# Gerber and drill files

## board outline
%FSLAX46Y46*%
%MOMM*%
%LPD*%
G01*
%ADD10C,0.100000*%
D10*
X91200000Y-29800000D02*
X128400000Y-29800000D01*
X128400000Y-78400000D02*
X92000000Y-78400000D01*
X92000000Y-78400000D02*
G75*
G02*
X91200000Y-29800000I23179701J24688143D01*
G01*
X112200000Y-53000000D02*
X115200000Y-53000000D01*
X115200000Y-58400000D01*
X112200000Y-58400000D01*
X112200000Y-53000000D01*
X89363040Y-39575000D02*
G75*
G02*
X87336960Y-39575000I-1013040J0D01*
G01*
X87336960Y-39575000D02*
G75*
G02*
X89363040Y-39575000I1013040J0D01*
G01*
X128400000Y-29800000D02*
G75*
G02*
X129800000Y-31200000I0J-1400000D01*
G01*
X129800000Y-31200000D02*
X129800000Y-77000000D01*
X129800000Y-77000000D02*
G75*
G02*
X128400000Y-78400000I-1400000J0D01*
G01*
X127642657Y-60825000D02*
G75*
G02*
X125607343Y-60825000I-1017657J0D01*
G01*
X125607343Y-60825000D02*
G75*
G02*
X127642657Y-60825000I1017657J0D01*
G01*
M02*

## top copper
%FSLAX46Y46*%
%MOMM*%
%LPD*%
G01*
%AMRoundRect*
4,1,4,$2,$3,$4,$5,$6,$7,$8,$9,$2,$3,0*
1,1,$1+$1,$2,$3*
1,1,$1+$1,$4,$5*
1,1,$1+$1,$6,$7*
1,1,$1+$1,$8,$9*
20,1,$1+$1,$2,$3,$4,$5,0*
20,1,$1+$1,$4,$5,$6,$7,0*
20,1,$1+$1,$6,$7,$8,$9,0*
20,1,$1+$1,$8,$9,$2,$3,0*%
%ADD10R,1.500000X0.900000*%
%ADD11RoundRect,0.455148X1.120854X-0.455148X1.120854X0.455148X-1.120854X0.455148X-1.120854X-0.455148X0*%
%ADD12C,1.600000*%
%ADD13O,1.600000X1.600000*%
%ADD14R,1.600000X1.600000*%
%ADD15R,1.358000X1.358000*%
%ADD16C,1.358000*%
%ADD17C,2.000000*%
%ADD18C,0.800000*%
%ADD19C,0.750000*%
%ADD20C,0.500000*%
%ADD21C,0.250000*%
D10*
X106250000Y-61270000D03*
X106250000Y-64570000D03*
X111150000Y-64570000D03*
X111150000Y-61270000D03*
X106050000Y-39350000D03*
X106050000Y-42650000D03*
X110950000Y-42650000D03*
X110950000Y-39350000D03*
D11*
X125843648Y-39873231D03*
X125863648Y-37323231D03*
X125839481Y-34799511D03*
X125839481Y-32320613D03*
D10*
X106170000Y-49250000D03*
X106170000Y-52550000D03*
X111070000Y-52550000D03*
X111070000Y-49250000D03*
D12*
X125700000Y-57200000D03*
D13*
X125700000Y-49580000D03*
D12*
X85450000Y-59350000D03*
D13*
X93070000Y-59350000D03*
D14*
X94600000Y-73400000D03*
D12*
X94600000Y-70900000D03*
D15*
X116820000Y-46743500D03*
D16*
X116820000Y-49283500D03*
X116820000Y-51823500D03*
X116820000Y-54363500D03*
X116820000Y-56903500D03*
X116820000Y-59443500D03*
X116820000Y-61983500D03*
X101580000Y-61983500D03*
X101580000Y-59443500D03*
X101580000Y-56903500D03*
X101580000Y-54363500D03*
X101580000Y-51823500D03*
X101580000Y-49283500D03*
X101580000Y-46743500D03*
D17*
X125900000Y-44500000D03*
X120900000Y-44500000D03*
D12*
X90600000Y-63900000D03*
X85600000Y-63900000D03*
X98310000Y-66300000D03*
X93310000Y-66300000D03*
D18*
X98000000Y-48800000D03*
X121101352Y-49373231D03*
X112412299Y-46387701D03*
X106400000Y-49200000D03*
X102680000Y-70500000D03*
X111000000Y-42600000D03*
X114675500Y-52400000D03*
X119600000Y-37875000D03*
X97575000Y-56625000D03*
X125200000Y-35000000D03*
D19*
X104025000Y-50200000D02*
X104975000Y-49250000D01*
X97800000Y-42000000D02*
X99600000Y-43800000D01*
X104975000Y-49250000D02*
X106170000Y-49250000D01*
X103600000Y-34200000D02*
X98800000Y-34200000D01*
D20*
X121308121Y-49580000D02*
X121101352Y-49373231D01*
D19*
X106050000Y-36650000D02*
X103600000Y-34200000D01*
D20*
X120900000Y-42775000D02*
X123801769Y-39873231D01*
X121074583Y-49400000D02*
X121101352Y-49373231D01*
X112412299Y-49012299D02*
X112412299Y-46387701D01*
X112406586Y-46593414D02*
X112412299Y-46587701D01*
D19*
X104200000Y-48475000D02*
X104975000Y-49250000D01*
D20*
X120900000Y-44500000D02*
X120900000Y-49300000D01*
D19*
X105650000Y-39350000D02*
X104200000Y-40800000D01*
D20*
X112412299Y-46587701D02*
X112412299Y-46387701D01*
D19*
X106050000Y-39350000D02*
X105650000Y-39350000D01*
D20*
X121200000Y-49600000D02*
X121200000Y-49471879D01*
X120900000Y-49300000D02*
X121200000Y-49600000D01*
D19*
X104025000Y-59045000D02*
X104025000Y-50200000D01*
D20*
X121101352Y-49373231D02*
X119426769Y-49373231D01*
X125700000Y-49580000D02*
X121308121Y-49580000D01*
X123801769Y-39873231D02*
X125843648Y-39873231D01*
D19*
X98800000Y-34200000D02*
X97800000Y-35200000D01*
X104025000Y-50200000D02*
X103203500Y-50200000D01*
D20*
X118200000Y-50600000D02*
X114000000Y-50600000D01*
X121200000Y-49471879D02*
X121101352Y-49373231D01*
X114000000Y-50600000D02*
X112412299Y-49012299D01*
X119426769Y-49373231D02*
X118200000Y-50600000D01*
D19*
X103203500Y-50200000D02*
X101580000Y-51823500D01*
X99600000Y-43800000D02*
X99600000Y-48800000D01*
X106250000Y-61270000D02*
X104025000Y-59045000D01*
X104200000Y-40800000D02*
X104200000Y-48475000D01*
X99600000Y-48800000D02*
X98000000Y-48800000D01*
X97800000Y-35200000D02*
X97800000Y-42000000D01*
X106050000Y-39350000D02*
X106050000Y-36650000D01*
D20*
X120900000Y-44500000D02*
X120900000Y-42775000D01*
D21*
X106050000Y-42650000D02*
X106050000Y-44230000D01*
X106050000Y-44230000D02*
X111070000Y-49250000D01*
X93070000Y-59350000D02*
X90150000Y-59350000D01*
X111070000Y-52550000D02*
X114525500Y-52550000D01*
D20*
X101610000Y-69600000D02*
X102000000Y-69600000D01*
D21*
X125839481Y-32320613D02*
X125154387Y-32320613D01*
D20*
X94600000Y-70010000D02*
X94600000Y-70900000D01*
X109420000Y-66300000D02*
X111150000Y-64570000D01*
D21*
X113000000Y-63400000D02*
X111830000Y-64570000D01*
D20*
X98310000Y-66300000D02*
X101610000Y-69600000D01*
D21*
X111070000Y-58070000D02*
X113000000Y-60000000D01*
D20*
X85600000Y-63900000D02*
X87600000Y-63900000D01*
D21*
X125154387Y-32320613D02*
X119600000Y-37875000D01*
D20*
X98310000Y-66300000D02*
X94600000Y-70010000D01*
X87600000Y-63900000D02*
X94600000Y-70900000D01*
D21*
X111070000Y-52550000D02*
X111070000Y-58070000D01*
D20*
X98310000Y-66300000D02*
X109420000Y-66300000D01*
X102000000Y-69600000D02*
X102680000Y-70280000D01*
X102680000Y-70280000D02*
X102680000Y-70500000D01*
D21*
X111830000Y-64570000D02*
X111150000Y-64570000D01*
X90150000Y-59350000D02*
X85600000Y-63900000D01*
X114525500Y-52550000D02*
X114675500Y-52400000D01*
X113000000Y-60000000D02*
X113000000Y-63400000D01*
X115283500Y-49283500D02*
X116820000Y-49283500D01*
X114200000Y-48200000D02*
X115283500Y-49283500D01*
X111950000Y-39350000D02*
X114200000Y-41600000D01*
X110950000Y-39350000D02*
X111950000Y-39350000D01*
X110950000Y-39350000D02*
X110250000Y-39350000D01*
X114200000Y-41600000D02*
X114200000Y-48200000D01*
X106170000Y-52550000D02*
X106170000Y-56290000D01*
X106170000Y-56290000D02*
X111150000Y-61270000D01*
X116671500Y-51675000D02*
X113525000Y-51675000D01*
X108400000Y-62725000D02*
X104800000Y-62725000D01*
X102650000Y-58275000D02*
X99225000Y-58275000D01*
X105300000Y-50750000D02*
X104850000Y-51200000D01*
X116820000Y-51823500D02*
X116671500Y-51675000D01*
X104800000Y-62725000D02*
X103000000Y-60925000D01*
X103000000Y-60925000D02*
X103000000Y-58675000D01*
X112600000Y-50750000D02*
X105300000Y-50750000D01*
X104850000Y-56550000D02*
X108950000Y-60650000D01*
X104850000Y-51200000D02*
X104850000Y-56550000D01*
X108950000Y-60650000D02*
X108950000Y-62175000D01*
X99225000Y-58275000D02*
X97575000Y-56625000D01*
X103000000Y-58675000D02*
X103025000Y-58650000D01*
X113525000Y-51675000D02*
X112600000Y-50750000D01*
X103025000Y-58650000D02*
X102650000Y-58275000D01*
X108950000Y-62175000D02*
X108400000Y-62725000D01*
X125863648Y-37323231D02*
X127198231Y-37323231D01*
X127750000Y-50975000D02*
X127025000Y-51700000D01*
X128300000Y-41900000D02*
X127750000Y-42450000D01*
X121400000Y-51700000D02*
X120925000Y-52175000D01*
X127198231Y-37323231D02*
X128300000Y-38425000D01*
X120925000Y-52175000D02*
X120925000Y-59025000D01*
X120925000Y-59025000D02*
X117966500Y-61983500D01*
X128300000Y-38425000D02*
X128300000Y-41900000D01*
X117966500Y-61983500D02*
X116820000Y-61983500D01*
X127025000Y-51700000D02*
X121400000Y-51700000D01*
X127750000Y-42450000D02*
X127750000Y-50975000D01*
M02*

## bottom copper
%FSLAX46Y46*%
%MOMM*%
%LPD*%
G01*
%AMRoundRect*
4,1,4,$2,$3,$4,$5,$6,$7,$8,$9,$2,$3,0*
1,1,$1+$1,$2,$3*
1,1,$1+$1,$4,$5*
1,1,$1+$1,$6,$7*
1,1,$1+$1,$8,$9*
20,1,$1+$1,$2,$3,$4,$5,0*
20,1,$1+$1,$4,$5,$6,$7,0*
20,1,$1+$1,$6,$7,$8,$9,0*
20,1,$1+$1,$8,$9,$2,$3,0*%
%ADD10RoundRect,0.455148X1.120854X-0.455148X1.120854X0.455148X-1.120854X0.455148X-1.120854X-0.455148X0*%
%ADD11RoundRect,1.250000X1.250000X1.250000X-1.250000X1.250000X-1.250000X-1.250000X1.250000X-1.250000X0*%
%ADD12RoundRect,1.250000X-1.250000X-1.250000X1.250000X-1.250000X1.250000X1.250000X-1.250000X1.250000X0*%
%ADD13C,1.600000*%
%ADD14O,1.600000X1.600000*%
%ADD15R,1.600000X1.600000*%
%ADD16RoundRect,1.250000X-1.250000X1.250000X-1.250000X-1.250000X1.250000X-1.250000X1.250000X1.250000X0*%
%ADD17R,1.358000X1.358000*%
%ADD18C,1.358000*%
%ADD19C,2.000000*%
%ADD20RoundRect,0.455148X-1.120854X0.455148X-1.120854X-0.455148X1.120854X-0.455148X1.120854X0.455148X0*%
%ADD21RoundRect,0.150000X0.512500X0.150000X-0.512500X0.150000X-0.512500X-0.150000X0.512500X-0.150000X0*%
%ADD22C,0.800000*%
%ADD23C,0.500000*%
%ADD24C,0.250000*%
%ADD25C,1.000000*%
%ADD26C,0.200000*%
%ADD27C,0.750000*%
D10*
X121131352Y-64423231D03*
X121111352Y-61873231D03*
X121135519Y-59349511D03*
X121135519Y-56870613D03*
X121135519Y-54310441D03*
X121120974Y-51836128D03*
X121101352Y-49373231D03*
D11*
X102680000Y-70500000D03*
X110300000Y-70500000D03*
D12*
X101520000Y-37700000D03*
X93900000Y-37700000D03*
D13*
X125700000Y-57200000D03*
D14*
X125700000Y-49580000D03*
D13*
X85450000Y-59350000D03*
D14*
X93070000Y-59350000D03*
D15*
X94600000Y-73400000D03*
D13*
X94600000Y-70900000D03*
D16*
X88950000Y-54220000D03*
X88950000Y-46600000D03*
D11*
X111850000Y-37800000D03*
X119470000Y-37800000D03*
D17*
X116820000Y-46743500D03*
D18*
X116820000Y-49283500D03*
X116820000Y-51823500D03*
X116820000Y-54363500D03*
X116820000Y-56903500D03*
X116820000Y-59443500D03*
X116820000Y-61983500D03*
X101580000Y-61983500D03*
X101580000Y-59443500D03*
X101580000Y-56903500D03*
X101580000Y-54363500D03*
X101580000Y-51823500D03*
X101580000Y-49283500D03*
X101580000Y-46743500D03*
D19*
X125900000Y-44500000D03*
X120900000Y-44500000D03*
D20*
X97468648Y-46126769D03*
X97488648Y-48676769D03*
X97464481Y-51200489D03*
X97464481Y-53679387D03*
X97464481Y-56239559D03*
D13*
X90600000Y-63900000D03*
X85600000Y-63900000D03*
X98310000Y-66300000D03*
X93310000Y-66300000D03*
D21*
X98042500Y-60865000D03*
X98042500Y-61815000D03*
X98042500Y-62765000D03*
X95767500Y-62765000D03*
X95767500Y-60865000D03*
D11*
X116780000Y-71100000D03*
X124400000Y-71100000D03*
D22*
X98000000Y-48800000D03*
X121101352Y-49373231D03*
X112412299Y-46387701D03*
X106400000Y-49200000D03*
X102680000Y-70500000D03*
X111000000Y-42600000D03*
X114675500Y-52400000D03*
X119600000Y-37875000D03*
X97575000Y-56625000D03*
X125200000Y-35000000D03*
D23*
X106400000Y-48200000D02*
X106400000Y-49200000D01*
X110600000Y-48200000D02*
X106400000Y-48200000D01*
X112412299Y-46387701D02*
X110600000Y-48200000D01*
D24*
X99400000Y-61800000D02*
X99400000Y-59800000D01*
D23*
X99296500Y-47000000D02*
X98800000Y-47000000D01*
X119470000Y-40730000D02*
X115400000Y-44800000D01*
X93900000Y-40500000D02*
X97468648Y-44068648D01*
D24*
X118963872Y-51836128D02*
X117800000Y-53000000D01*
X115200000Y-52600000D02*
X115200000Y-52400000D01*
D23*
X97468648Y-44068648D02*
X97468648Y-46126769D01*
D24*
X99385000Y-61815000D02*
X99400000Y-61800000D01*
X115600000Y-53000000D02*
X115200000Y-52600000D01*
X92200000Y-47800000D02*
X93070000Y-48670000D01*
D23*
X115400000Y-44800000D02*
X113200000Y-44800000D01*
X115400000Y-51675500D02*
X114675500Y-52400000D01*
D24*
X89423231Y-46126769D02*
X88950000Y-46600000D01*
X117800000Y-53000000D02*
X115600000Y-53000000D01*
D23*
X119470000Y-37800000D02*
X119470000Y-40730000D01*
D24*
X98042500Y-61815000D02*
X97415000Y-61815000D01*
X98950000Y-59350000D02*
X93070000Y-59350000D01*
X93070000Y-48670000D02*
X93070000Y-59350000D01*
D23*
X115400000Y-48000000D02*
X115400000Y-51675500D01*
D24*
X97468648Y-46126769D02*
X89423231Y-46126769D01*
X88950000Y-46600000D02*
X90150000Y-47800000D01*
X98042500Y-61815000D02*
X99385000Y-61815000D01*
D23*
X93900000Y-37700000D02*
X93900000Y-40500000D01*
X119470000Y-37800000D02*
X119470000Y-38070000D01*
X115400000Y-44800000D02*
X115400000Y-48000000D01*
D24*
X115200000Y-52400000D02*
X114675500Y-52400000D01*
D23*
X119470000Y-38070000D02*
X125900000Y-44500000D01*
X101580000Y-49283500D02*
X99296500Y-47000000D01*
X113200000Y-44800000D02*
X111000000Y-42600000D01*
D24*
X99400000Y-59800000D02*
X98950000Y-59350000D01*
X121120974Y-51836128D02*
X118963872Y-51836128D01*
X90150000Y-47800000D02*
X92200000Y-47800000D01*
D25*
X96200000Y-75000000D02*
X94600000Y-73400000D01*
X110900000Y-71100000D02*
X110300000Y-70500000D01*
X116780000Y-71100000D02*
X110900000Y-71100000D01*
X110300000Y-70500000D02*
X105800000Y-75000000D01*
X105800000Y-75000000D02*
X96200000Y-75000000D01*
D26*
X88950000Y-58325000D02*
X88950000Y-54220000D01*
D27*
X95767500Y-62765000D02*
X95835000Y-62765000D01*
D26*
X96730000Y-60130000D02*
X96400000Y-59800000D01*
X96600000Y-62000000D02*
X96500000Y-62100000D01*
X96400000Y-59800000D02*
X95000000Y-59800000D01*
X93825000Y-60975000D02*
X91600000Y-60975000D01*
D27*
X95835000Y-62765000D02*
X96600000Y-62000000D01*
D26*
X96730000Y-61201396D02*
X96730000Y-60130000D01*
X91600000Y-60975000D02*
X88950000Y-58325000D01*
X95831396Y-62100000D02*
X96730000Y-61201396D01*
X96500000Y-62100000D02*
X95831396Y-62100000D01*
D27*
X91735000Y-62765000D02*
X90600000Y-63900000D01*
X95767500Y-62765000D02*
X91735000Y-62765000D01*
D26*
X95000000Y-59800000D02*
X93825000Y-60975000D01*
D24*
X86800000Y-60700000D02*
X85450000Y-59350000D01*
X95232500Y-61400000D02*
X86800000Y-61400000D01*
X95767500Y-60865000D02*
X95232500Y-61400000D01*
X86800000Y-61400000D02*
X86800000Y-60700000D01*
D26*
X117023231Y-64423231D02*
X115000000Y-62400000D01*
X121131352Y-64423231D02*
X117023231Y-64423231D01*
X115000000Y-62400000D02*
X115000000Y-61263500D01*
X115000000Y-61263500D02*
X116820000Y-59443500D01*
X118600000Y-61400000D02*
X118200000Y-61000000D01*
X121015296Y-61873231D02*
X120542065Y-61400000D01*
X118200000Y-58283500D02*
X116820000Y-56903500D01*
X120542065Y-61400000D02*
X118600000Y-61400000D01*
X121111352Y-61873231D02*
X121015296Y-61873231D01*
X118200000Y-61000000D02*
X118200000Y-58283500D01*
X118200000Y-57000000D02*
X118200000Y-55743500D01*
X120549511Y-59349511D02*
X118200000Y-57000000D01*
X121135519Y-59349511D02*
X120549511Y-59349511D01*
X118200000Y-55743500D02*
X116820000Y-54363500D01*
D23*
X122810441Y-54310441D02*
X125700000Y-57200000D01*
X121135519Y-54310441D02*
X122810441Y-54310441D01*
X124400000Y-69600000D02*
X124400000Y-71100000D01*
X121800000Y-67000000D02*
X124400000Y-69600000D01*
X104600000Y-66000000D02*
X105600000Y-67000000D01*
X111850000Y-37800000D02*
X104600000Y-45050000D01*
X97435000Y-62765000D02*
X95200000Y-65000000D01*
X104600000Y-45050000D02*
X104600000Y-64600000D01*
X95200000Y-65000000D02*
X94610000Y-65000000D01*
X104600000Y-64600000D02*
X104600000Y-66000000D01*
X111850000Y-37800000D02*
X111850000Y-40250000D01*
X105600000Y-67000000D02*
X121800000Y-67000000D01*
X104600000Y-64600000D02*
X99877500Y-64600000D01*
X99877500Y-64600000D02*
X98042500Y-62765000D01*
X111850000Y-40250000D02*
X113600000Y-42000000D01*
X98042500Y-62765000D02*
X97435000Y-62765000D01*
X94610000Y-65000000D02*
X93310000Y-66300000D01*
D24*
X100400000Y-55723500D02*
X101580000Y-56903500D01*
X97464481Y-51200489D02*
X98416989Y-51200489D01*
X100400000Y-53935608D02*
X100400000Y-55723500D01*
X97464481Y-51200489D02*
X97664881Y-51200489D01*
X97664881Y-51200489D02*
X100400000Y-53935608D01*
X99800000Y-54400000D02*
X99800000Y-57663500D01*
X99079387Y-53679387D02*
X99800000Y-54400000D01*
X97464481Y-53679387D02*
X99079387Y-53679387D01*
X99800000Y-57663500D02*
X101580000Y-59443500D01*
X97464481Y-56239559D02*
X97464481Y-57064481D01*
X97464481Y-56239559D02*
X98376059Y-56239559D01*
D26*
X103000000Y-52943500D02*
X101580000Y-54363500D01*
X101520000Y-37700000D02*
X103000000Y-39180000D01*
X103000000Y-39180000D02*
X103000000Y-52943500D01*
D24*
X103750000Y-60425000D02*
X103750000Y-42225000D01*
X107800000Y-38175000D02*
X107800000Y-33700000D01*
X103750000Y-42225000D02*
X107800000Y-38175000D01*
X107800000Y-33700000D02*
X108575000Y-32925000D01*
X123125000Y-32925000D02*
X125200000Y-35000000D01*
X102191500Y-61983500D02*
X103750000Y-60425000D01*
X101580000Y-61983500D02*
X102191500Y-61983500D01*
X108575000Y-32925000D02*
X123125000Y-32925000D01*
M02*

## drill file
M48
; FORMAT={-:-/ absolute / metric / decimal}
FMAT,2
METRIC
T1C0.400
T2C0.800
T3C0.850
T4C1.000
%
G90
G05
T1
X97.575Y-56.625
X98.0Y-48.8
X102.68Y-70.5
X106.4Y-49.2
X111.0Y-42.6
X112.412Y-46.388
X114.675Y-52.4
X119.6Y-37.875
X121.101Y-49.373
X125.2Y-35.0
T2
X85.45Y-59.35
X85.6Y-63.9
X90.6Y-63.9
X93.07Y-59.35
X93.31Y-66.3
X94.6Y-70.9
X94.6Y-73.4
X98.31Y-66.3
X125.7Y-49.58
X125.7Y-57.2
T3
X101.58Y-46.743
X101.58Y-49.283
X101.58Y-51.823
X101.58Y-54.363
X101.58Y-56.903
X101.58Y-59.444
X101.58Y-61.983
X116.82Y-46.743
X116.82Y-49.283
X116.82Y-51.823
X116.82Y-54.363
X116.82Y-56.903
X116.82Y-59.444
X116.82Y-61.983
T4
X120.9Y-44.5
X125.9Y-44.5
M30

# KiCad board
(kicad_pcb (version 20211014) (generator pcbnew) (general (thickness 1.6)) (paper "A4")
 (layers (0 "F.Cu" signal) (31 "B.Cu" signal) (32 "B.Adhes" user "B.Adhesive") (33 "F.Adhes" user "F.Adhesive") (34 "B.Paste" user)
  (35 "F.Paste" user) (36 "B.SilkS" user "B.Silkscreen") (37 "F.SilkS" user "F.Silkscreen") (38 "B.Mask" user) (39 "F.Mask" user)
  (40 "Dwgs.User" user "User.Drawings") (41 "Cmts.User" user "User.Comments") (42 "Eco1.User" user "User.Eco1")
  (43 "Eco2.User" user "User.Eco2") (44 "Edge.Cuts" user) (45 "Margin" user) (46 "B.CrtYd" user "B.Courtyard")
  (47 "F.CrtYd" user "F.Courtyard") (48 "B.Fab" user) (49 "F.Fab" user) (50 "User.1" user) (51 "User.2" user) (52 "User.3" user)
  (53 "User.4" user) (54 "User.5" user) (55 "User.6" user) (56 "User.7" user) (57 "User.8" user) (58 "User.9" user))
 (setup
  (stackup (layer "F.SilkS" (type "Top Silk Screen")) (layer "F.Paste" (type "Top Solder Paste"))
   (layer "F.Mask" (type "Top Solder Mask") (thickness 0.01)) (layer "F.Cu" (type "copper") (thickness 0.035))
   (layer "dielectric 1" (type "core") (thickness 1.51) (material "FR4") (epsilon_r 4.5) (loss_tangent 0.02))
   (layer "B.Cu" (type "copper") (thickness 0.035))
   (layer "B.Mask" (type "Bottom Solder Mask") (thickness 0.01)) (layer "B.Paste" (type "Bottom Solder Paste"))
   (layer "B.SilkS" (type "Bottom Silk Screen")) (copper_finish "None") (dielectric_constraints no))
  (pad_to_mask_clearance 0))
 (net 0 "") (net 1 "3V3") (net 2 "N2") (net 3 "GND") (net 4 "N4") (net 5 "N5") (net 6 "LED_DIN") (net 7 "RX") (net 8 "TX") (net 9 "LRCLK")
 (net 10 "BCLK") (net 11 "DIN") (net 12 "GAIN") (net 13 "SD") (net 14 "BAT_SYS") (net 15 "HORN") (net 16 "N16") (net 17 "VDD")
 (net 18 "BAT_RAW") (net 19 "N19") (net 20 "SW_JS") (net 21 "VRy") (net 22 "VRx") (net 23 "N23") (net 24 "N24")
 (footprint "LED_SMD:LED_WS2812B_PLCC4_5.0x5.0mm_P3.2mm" (layer "F.Cu") (at 108.7 62.92)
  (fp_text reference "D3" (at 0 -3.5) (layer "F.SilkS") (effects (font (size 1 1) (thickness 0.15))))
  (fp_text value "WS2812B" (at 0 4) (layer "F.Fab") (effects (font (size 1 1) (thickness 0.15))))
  (pad "1" smd rect (at -2.45 -1.65) (size 1.5 0.9) (layers "F.Cu" "F.Paste" "F.Mask") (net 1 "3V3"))
  (pad "2" smd rect (at -2.45 1.65) (size 1.5 0.9) (layers "F.Cu" "F.Paste" "F.Mask") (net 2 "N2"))
  (pad "3" smd rect (at 2.45 1.65) (size 1.5 0.9) (layers "F.Cu" "F.Paste" "F.Mask") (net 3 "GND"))
  (pad "4" smd rect (at 2.45 -1.65) (size 1.5 0.9) (layers "F.Cu" "F.Paste" "F.Mask") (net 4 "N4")))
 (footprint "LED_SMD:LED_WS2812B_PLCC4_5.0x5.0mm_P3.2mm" (layer "F.Cu") (at 108.5 41)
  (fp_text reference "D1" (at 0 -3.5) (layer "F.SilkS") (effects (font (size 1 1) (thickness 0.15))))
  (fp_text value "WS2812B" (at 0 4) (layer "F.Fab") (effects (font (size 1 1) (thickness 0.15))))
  (pad "1" smd rect (at -2.45 -1.65) (size 1.5 0.9) (layers "F.Cu" "F.Paste" "F.Mask") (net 1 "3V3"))
  (pad "2" smd rect (at -2.45 1.65) (size 1.5 0.9) (layers "F.Cu" "F.Paste" "F.Mask") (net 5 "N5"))
  (pad "3" smd rect (at 2.45 1.65) (size 1.5 0.9) (layers "F.Cu" "F.Paste" "F.Mask") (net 3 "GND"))
  (pad "4" smd rect (at 2.45 -1.65) (size 1.5 0.9) (layers "F.Cu" "F.Paste" "F.Mask") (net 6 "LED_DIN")))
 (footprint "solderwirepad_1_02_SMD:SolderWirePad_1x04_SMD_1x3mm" (layer "F.Cu") (at 125.875 39.85 90)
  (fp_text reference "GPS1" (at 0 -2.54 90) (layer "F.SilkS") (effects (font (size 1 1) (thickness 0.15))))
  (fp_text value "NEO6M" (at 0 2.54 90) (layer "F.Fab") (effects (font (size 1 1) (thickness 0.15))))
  (pad "1" smd roundrect (at -0.023231 -0.031352 90) (size 1.820592 3.152005) (layers "F.Cu" "F.Paste" "F.Mask") (roundrect_rratio 0.25)
   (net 1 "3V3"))
  (pad "2" smd roundrect (at 2.526769 -0.011352 90) (size 1.820592 3.152005) (layers "F.Cu" "F.Paste" "F.Mask") (roundrect_rratio 0.25)
   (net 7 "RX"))
  (pad "3" smd roundrect (at 5.050489 -0.035519 90) (size 1.820592 3.152005) (layers "F.Cu" "F.Paste" "F.Mask") (roundrect_rratio 0.25)
   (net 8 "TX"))
  (pad "4" smd roundrect (at 7.529387 -0.035519 90) (size 1.820592 3.152005) (layers "F.Cu" "F.Paste" "F.Mask") (roundrect_rratio 0.25)
   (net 3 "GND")))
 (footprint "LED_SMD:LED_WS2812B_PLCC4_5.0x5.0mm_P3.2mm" (layer "F.Cu") (at 108.62 50.9)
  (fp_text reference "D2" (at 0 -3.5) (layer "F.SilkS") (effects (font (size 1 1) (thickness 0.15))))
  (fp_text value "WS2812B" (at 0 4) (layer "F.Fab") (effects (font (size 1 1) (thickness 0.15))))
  (pad "1" smd rect (at -2.45 -1.65) (size 1.5 0.9) (layers "F.Cu" "F.Paste" "F.Mask") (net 1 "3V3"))
  (pad "2" smd rect (at -2.45 1.65) (size 1.5 0.9) (layers "F.Cu" "F.Paste" "F.Mask") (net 4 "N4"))
  (pad "3" smd rect (at 2.45 1.65) (size 1.5 0.9) (layers "F.Cu" "F.Paste" "F.Mask") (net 3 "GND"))
  (pad "4" smd rect (at 2.45 -1.65) (size 1.5 0.9) (layers "F.Cu" "F.Paste" "F.Mask") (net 5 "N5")))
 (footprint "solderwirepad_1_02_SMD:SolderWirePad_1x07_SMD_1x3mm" (layer "B.Cu") (at 121.1 64.4 90)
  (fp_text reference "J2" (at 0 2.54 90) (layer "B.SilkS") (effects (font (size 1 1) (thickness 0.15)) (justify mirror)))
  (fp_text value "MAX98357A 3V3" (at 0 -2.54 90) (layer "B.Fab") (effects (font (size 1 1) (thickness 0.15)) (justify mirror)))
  (pad "1" smd roundrect (at -0.023231 0.031352 90) (size 1.820592 3.152005) (layers "B.Cu" "B.Paste" "B.Mask") (roundrect_rratio 0.25)
   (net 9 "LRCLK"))
  (pad "2" smd roundrect (at 2.526769 0.011352 90) (size 1.820592 3.152005) (layers "B.Cu" "B.Paste" "B.Mask") (roundrect_rratio 0.25)
   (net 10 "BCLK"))
  (pad "3" smd roundrect (at 5.050489 0.035519 90) (size 1.820592 3.152005) (layers "B.Cu" "B.Paste" "B.Mask") (roundrect_rratio 0.25)
   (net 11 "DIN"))
  (pad "4" smd roundrect (at 7.529387 0.035519 90) (size 1.820592 3.152005) (layers "B.Cu" "B.Paste" "B.Mask") (roundrect_rratio 0.25)
   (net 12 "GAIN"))
  (pad "5" smd roundrect (at 10.089559 0.035519 90) (size 1.820592 3.152005) (layers "B.Cu" "B.Paste" "B.Mask") (roundrect_rratio 0.25)
   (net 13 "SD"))
  (pad "6" smd roundrect (at 12.563872 0.020974 90) (size 1.820592 3.152005) (layers "B.Cu" "B.Paste" "B.Mask") (roundrect_rratio 0.25)
   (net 3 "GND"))
  (pad "7" smd roundrect (at 15.026769 0.001352 90) (size 1.820592 3.152005) (layers "B.Cu" "B.Paste" "B.Mask") (roundrect_rratio 0.25)
   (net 1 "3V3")))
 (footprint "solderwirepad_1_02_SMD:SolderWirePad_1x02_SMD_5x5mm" (layer "B.Cu") (at 110.3 70.5 180)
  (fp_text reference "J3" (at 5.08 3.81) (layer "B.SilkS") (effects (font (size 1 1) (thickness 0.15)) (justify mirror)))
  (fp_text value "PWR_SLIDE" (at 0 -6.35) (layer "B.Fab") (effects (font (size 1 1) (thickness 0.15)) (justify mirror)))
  (pad "1" smd roundrect (at 7.62 0 180) (size 5 5) (layers "B.Cu" "B.Paste" "B.Mask") (roundrect_rratio 0.25) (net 3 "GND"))
  (pad "2" smd roundrect (at 0 0 180) (size 5 5) (layers "B.Cu" "B.Paste" "B.Mask") (roundrect_rratio 0.25) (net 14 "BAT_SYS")))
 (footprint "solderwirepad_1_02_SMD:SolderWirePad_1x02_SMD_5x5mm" (layer "B.Cu") (at 93.9 37.7)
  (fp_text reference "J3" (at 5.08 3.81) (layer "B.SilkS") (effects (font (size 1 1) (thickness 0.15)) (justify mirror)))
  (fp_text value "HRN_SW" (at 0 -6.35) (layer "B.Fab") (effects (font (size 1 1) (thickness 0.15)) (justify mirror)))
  (pad "1" smd roundrect (at 7.62 0) (size 5 5) (layers "B.Cu" "B.Paste" "B.Mask") (roundrect_rratio 0.25) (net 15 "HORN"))
  (pad "2" smd roundrect (at 0 0) (size 5 5) (layers "B.Cu" "B.Paste" "B.Mask") (roundrect_rratio 0.25) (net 3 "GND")))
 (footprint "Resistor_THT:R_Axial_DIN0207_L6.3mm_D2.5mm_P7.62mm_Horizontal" (layer "B.Cu") (at 125.7 57.2 90)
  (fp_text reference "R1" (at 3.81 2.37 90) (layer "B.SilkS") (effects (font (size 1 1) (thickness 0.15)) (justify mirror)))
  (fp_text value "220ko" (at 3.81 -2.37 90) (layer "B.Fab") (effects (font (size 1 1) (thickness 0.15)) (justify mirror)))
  (pad "1" thru_hole circle (at 0 0 90) (size 1.6 1.6) (drill 0.8) (layers *.Cu *.Mask) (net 13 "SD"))
  (pad "2" thru_hole oval (at 7.62 0 90) (size 1.6 1.6) (drill 0.8) (layers *.Cu *.Mask) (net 1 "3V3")))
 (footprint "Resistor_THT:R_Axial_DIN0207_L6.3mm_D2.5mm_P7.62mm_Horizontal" (layer "B.Cu") (at 85.45 59.35)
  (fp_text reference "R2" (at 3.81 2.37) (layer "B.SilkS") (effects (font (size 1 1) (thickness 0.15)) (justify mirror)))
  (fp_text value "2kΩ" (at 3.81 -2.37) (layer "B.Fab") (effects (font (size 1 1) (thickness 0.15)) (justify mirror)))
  (pad "1" thru_hole circle (at 0 0) (size 1.6 1.6) (drill 0.8) (layers *.Cu *.Mask) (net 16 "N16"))
  (pad "2" thru_hole oval (at 7.62 0) (size 1.6 1.6) (drill 0.8) (layers *.Cu *.Mask) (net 3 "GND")))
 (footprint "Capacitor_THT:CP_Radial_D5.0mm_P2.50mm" (layer "B.Cu") (at 94.6 73.4 90)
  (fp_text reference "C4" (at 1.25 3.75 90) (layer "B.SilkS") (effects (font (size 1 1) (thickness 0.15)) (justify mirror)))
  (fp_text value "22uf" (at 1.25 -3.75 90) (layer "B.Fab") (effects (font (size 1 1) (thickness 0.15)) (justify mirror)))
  (pad "1" thru_hole rect (at 0 0 90) (size 1.6 1.6) (drill 0.8) (layers *.Cu *.Mask) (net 14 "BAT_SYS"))
  (pad "2" thru_hole circle (at 2.5 0 90) (size 1.6 1.6) (drill 0.8) (layers *.Cu *.Mask) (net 3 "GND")))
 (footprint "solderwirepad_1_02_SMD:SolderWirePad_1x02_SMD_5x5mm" (layer "B.Cu") (at 88.95 46.6 -90)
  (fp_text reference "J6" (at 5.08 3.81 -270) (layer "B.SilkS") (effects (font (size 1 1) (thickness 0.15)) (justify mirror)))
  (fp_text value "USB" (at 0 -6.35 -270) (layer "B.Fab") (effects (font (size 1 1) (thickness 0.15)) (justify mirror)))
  (pad "1" smd roundrect (at 7.62 0 270) (size 5 5) (layers "B.Cu" "B.Paste" "B.Mask") (roundrect_rratio 0.25) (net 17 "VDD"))
  (pad "2" smd roundrect (at 0 0 270) (size 5 5) (layers "B.Cu" "B.Paste" "B.Mask") (roundrect_rratio 0.25) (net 3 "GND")))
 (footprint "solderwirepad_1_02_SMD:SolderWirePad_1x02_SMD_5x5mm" (layer "B.Cu") (at 119.47 37.8 180)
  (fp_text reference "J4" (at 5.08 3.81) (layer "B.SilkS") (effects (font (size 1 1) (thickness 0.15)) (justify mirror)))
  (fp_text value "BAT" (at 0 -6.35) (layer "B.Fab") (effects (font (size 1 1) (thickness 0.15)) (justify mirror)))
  (pad "1" smd roundrect (at 7.62 0 180) (size 5 5) (layers "B.Cu" "B.Paste" "B.Mask") (roundrect_rratio 0.25) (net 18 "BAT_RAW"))
  (pad "2" smd roundrect (at 0 0 180) (size 5 5) (layers "B.Cu" "B.Paste" "B.Mask") (roundrect_rratio 0.25) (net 3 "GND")))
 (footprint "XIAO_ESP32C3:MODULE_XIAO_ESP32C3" (layer "B.Cu") (at 109.2 54.3 180)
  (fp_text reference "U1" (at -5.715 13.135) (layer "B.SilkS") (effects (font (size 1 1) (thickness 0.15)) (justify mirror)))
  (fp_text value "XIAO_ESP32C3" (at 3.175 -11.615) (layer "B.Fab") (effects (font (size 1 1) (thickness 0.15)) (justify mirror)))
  (pad "1" thru_hole rect (at -7.62 7.5565 180) (size 1.358 1.358) (drill 0.85) (layers *.Cu *.Mask) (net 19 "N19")
   (solder_mask_margin 0.102))
  (pad "2" thru_hole circle (at -7.62 5.0165 180) (size 1.358 1.358) (drill 0.85) (layers *.Cu *.Mask) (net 6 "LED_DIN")
   (solder_mask_margin 0.102))
  (pad "3" thru_hole circle (at -7.62 2.4765 180) (size 1.358 1.358) (drill 0.85) (layers *.Cu *.Mask) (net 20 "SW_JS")
   (solder_mask_margin 0.102))
  (pad "4" thru_hole circle (at -7.62 -0.0635 180) (size 1.358 1.358) (drill 0.85) (layers *.Cu *.Mask) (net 11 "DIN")
   (solder_mask_margin 0.102))
  (pad "5" thru_hole circle (at -7.62 -2.6035 180) (size 1.358 1.358) (drill 0.85) (layers *.Cu *.Mask) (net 10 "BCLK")
   (solder_mask_margin 0.102))
  (pad "6" thru_hole circle (at -7.62 -5.1435 180) (size 1.358 1.358) (drill 0.85) (layers *.Cu *.Mask) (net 9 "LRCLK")
   (solder_mask_margin 0.102))
  (pad "7" thru_hole circle (at -7.62 -7.6835 180) (size 1.358 1.358) (drill 0.85) (layers *.Cu *.Mask) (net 7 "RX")
   (solder_mask_margin 0.102))
  (pad "8" thru_hole circle (at 7.62 -7.6835 180) (size 1.358 1.358) (drill 0.85) (layers *.Cu *.Mask) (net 8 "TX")
   (solder_mask_margin 0.102))
  (pad "9" thru_hole circle (at 7.62 -5.1435 180) (size 1.358 1.358) (drill 0.85) (layers *.Cu *.Mask) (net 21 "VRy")
   (solder_mask_margin 0.102))
  (pad "10" thru_hole circle (at 7.62 -2.6035 180) (size 1.358 1.358) (drill 0.85) (layers *.Cu *.Mask) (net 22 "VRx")
   (solder_mask_margin 0.102))
  (pad "11" thru_hole circle (at 7.62 -0.0635 180) (size 1.358 1.358) (drill 0.85) (layers *.Cu *.Mask) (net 15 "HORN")
   (solder_mask_margin 0.102))
  (pad "12" thru_hole circle (at 7.62 2.4765 180) (size 1.358 1.358) (drill 0.85) (layers *.Cu *.Mask) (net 1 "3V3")
   (solder_mask_margin 0.102))
  (pad "13" thru_hole circle (at 7.62 5.0165 180) (size 1.358 1.358) (drill 0.85) (layers *.Cu *.Mask) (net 3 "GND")
   (solder_mask_margin 0.102))
  (pad "14" thru_hole circle (at 7.62 7.5565 180) (size 1.358 1.358) (drill 0.85) (layers *.Cu *.Mask) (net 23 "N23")
   (solder_mask_margin 0.102)))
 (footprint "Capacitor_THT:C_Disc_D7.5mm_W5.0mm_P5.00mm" (layer "B.Cu") (at 125.9 44.5 180)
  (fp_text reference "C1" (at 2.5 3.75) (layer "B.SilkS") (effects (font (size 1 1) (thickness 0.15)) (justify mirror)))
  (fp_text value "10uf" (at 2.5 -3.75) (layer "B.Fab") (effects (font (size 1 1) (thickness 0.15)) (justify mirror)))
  (pad "1" thru_hole circle (at 0 0 180) (size 2 2) (drill 1) (layers *.Cu *.Mask) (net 3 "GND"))
  (pad "2" thru_hole circle (at 5 0 180) (size 2 2) (drill 1) (layers *.Cu *.Mask) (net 1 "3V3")))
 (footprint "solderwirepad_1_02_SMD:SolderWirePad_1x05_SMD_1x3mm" (layer "B.Cu") (at 97.5 46.15 -90)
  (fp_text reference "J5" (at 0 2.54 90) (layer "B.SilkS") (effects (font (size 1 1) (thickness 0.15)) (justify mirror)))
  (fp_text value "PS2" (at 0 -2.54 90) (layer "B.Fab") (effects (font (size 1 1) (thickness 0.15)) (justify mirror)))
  (pad "1" smd roundrect (at -0.023231 0.031352 270) (size 1.820592 3.152005) (layers "B.Cu" "B.Paste" "B.Mask") (roundrect_rratio 0.25)
   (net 3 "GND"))
  (pad "2" smd roundrect (at 2.526769 0.011352 270) (size 1.820592 3.152005) (layers "B.Cu" "B.Paste" "B.Mask") (roundrect_rratio 0.25)
   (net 1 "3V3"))
  (pad "3" smd roundrect (at 5.050489 0.035519 270) (size 1.820592 3.152005) (layers "B.Cu" "B.Paste" "B.Mask") (roundrect_rratio 0.25)
   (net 22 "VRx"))
  (pad "4" smd roundrect (at 7.529387 0.035519 270) (size 1.820592 3.152005) (layers "B.Cu" "B.Paste" "B.Mask") (roundrect_rratio 0.25)
   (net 21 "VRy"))
  (pad "5" smd roundrect (at 10.089559 0.035519 270) (size 1.820592 3.152005) (layers "B.Cu" "B.Paste" "B.Mask") (roundrect_rratio 0.25)
   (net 20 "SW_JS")))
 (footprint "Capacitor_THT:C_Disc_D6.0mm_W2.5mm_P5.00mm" (layer "B.Cu") (at 90.6 63.9 180)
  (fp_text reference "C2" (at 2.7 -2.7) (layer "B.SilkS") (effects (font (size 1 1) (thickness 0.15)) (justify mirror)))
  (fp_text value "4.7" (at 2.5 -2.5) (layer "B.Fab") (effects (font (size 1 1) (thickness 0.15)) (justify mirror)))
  (pad "1" thru_hole circle (at 0 0 180) (size 1.6 1.6) (drill 0.8) (layers *.Cu *.Mask) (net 17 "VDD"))
  (pad "2" thru_hole circle (at 5 0 180) (size 1.6 1.6) (drill 0.8) (layers *.Cu *.Mask) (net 3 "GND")))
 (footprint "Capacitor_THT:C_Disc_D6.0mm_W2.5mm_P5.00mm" (layer "B.Cu") (at 98.31 66.3 180)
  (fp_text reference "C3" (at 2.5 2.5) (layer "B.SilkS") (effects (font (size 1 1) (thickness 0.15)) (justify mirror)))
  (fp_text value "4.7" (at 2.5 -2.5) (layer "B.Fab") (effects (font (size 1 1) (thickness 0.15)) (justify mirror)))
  (pad "1" thru_hole circle (at 0 0 180) (size 1.6 1.6) (drill 0.8) (layers *.Cu *.Mask) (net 3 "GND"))
  (pad "2" thru_hole circle (at 5 0 180) (size 1.6 1.6) (drill 0.8) (layers *.Cu *.Mask) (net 18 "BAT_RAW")))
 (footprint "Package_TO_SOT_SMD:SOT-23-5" (layer "B.Cu") (at 96.905 61.815 180)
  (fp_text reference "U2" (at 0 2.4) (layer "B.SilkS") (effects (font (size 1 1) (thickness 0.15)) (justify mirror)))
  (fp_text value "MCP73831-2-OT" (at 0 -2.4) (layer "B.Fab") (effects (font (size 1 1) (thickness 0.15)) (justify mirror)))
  (pad "1" smd roundrect (at -1.1375 0.95 180) (size 1.325 0.6) (layers "B.Cu" "B.Paste" "B.Mask") (roundrect_rratio 0.25) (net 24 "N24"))
  (pad "2" smd roundrect (at -1.1375 0 180) (size 1.325 0.6) (layers "B.Cu" "B.Paste" "B.Mask") (roundrect_rratio 0.25) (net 3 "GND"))
  (pad "3" smd roundrect (at -1.1375 -0.95 180) (size 1.325 0.6) (layers "B.Cu" "B.Paste" "B.Mask") (roundrect_rratio 0.25)
   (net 18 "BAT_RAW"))
  (pad "4" smd roundrect (at 1.1375 -0.95 180) (size 1.325 0.6) (layers "B.Cu" "B.Paste" "B.Mask") (roundrect_rratio 0.25) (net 17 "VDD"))
  (pad "5" smd roundrect (at 1.1375 0.95 180) (size 1.325 0.6) (layers "B.Cu" "B.Paste" "B.Mask") (roundrect_rratio 0.25) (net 16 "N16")))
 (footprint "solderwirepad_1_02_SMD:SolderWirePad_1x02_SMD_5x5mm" (layer "B.Cu") (at 124.4 71.1 180)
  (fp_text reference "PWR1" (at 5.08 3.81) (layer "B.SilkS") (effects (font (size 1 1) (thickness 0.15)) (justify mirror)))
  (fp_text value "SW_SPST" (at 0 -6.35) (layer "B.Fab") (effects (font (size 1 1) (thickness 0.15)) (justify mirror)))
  (pad "1" smd roundrect (at 7.62 0 180) (size 5 5) (layers "B.Cu" "B.Paste" "B.Mask") (roundrect_rratio 0.25) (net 14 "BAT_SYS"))
  (pad "2" smd roundrect (at 0 0 180) (size 5 5) (layers "B.Cu" "B.Paste" "B.Mask") (roundrect_rratio 0.25) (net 18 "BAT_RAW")))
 (gr_line (start 91.2 29.8) (end 128.4 29.8) (layer "Edge.Cuts") (width 0.1))
 (gr_line (start 128.4 78.4) (end 92 78.4) (layer "Edge.Cuts") (width 0.1))
 (gr_arc (start 92 78.4) (mid 81.319809 54.269224) (end 91.2 29.8) (layer "Edge.Cuts") (width 0.1))
 (gr_rect (start 112.2 53) (end 115.2 58.4) (layer "Edge.Cuts") (width 0.1) (fill none))
 (gr_circle (center 88.35 39.575) (end 88.075 40.55) (layer "Edge.Cuts") (width 0.1) (fill none))
 (gr_arc (start 128.4 29.8) (mid 129.389949 30.210051) (end 129.8 31.2) (layer "Edge.Cuts") (width 0.1))
 (gr_line (start 129.8 31.2) (end 129.8 77) (layer "Edge.Cuts") (width 0.1))
 (gr_arc (start 129.8 77) (mid 129.389949 77.989949) (end 128.4 78.4) (layer "Edge.Cuts") (width 0.1))
 (gr_circle (center 126.625 60.825) (end 126.15 61.725) (layer "Edge.Cuts") (width 0.1) (fill none))
 (segment (start 104.025 50.2) (end 104.975 49.25) (width 0.75) (layer "F.Cu") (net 1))
 (segment (start 97.8 42) (end 99.6 43.8) (width 0.75) (layer "F.Cu") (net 1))
 (segment (start 104.975 49.25) (end 106.17 49.25) (width 0.75) (layer "F.Cu") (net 1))
 (segment (start 103.6 34.2) (end 98.8 34.2) (width 0.75) (layer "F.Cu") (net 1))
 (segment (start 121.308121 49.58) (end 121.101352 49.373231) (width 0.5) (layer "F.Cu") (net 1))
 (segment (start 106.05 36.65) (end 103.6 34.2) (width 0.75) (layer "F.Cu") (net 1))
 (segment (start 120.9 42.775) (end 123.801769 39.873231) (width 0.5) (layer "F.Cu") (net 1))
 (segment (start 121.074583 49.4) (end 121.101352 49.373231) (width 0.5) (layer "F.Cu") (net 1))
 (segment (start 112.412299 49.012299) (end 112.412299 46.387701) (width 0.5) (layer "F.Cu") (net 1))
 (segment (start 112.406586 46.593414) (end 112.412299 46.587701) (width 0.5) (layer "F.Cu") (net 1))
 (segment (start 104.2 48.475) (end 104.975 49.25) (width 0.75) (layer "F.Cu") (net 1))
 (segment (start 120.9 44.5) (end 120.9 49.3) (width 0.5) (layer "F.Cu") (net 1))
 (segment (start 105.65 39.35) (end 104.2 40.8) (width 0.75) (layer "F.Cu") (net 1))
 (segment (start 112.412299 46.587701) (end 112.412299 46.387701) (width 0.5) (layer "F.Cu") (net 1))
 (segment (start 106.05 39.35) (end 105.65 39.35) (width 0.75) (layer "F.Cu") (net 1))
 (segment (start 121.2 49.6) (end 121.2 49.471879) (width 0.5) (layer "F.Cu") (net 1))
 (segment (start 120.9 49.3) (end 121.2 49.6) (width 0.5) (layer "F.Cu") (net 1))
 (segment (start 104.025 59.045) (end 104.025 50.2) (width 0.75) (layer "F.Cu") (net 1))
 (segment (start 121.101352 49.373231) (end 119.426769 49.373231) (width 0.5) (layer "F.Cu") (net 1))
 (segment (start 125.7 49.58) (end 121.308121 49.58) (width 0.5) (layer "F.Cu") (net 1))
 (segment (start 123.801769 39.873231) (end 125.843648 39.873231) (width 0.5) (layer "F.Cu") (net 1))
 (segment (start 98.8 34.2) (end 97.8 35.2) (width 0.75) (layer "F.Cu") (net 1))
 (segment (start 104.025 50.2) (end 103.2035 50.2) (width 0.75) (layer "F.Cu") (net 1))
 (segment (start 118.2 50.6) (end 114 50.6) (width 0.5) (layer "F.Cu") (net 1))
 (segment (start 121.2 49.471879) (end 121.101352 49.373231) (width 0.5) (layer "F.Cu") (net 1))
 (segment (start 114 50.6) (end 112.412299 49.012299) (width 0.5) (layer "F.Cu") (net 1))
 (segment (start 119.426769 49.373231) (end 118.2 50.6) (width 0.5) (layer "F.Cu") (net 1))
 (segment (start 103.2035 50.2) (end 101.58 51.8235) (width 0.75) (layer "F.Cu") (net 1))
 (segment (start 99.6 43.8) (end 99.6 48.8) (width 0.75) (layer "F.Cu") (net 1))
 (segment (start 106.25 61.27) (end 104.025 59.045) (width 0.75) (layer "F.Cu") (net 1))
 (segment (start 104.2 40.8) (end 104.2 48.475) (width 0.75) (layer "F.Cu") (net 1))
 (segment (start 99.6 48.8) (end 98 48.8) (width 0.75) (layer "F.Cu") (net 1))
 (segment (start 97.8 35.2) (end 97.8 42) (width 0.75) (layer "F.Cu") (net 1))
 (segment (start 106.05 39.35) (end 106.05 36.65) (width 0.75) (layer "F.Cu") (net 1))
 (segment (start 120.9 44.5) (end 120.9 42.775) (width 0.5) (layer "F.Cu") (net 1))
 (via (at 98 48.8) (size 0.8) (drill 0.4) (layers "F.Cu" "B.Cu") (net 1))
 (via (at 121.101352 49.373231) (size 0.8) (drill 0.4) (layers "F.Cu" "B.Cu") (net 1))
 (via (at 112.412299 46.387701) (size 0.8) (drill 0.4) (layers "F.Cu" "B.Cu") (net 1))
 (via (at 106.4 49.2) (size 0.8) (drill 0.4) (layers "F.Cu" "B.Cu") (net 1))
 (segment (start 106.4 48.2) (end 106.4 49.2) (width 0.5) (layer "B.Cu") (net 1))
 (segment (start 110.6 48.2) (end 106.4 48.2) (width 0.5) (layer "B.Cu") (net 1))
 (segment (start 112.412299 46.387701) (end 110.6 48.2) (width 0.5) (layer "B.Cu") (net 1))
 (segment (start 106.05 42.65) (end 106.05 44.23) (width 0.25) (layer "F.Cu") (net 5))
 (segment (start 106.05 44.23) (end 111.07 49.25) (width 0.25) (layer "F.Cu") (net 5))
 (segment (start 93.07 59.35) (end 90.15 59.35) (width 0.25) (layer "F.Cu") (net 3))
 (segment (start 111.07 52.55) (end 114.5255 52.55) (width 0.25) (layer "F.Cu") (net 3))
 (segment (start 101.61 69.6) (end 102 69.6) (width 0.5) (layer "F.Cu") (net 3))
 (segment (start 125.839481 32.320613) (end 125.154387 32.320613) (width 0.25) (layer "F.Cu") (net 3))
 (segment (start 94.6 70.01) (end 94.6 70.9) (width 0.5) (layer "F.Cu") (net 3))
 (segment (start 109.42 66.3) (end 111.15 64.57) (width 0.5) (layer "F.Cu") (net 3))
 (segment (start 113 63.4) (end 111.83 64.57) (width 0.25) (layer "F.Cu") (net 3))
 (segment (start 98.31 66.3) (end 101.61 69.6) (width 0.5) (layer "F.Cu") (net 3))
 (segment (start 111.07 58.07) (end 113 60) (width 0.25) (layer "F.Cu") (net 3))
 (segment (start 85.6 63.9) (end 87.6 63.9) (width 0.5) (layer "F.Cu") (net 3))
 (segment (start 125.154387 32.320613) (end 119.6 37.875) (width 0.25) (layer "F.Cu") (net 3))
 (segment (start 98.31 66.3) (end 94.6 70.01) (width 0.5) (layer "F.Cu") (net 3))
 (segment (start 87.6 63.9) (end 94.6 70.9) (width 0.5) (layer "F.Cu") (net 3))
 (segment (start 111.07 52.55) (end 111.07 58.07) (width 0.25) (layer "F.Cu") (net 3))
 (segment (start 98.31 66.3) (end 109.42 66.3) (width 0.5) (layer "F.Cu") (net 3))
 (segment (start 102 69.6) (end 102.68 70.28) (width 0.5) (layer "F.Cu") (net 3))
 (segment (start 102.68 70.28) (end 102.68 70.5) (width 0.5) (layer "F.Cu") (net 3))
 (segment (start 111.83 64.57) (end 111.15 64.57) (width 0.25) (layer "F.Cu") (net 3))
 (segment (start 90.15 59.35) (end 85.6 63.9) (width 0.25) (layer "F.Cu") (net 3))
 (segment (start 114.5255 52.55) (end 114.6755 52.4) (width 0.25) (layer "F.Cu") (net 3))
 (segment (start 113 60) (end 113 63.4) (width 0.25) (layer "F.Cu") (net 3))
 (via (at 102.68 70.5) (size 0.8) (drill 0.4) (layers "F.Cu" "B.Cu") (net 3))
 (via (at 111 42.6) (size 0.8) (drill 0.4) (layers "F.Cu" "B.Cu") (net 3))
 (via (at 114.6755 52.4) (size 0.8) (drill 0.4) (layers "F.Cu" "B.Cu") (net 3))
 (via (at 119.6 37.875) (size 0.8) (drill 0.4) (layers "F.Cu" "B.Cu") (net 3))
 (segment (start 99.4 61.8) (end 99.4 59.8) (width 0.25) (layer "B.Cu") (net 3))
 (segment (start 99.2965 47) (end 98.8 47) (width 0.5) (layer "B.Cu") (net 3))
 (segment (start 119.47 40.73) (end 115.4 44.8) (width 0.5) (layer "B.Cu") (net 3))
 (segment (start 93.9 40.5) (end 97.468648 44.068648) (width 0.5) (layer "B.Cu") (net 3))
 (segment (start 118.963872 51.836128) (end 117.8 53) (width 0.25) (layer "B.Cu") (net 3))
 (segment (start 115.2 52.6) (end 115.2 52.4) (width 0.25) (layer "B.Cu") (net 3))
 (segment (start 97.468648 44.068648) (end 97.468648 46.126769) (width 0.5) (layer "B.Cu") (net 3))
 (segment (start 99.385 61.815) (end 99.4 61.8) (width 0.25) (layer "B.Cu") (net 3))
 (segment (start 115.6 53) (end 115.2 52.6) (width 0.25) (layer "B.Cu") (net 3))
 (segment (start 92.2 47.8) (end 93.07 48.67) (width 0.25) (layer "B.Cu") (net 3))
 (segment (start 115.4 44.8) (end 113.2 44.8) (width 0.5) (layer "B.Cu") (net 3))
 (segment (start 115.4 51.6755) (end 114.6755 52.4) (width 0.5) (layer "B.Cu") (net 3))
 (segment (start 89.423231 46.126769) (end 88.95 46.6) (width 0.25) (layer "B.Cu") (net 3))
 (segment (start 117.8 53) (end 115.6 53) (width 0.25) (layer "B.Cu") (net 3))
 (segment (start 119.47 37.8) (end 119.47 40.73) (width 0.5) (layer "B.Cu") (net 3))
 (segment (start 98.0425 61.815) (end 97.415 61.815) (width 0.25) (layer "B.Cu") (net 3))
 (segment (start 98.95 59.35) (end 93.07 59.35) (width 0.25) (layer "B.Cu") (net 3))
 (segment (start 93.07 48.67) (end 93.07 59.35) (width 0.25) (layer "B.Cu") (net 3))
 (segment (start 115.4 48) (end 115.4 51.6755) (width 0.5) (layer "B.Cu") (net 3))
 (segment (start 97.468648 46.126769) (end 89.423231 46.126769) (width 0.25) (layer "B.Cu") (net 3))
 (segment (start 88.95 46.6) (end 90.15 47.8) (width 0.25) (layer "B.Cu") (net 3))
 (segment (start 98.0425 61.815) (end 99.385 61.815) (width 0.25) (layer "B.Cu") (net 3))
 (segment (start 93.9 37.7) (end 93.9 40.5) (width 0.5) (layer "B.Cu") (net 3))
 (segment (start 119.47 37.8) (end 119.47 38.07) (width 0.5) (layer "B.Cu") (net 3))
 (segment (start 115.4 44.8) (end 115.4 48) (width 0.5) (layer "B.Cu") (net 3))
 (segment (start 115.2 52.4) (end 114.6755 52.4) (width 0.25) (layer "B.Cu") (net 3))
 (segment (start 119.47 38.07) (end 125.9 44.5) (width 0.5) (layer "B.Cu") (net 3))
 (segment (start 101.58 49.2835) (end 99.2965 47) (width 0.5) (layer "B.Cu") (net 3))
 (segment (start 113.2 44.8) (end 111 42.6) (width 0.5) (layer "B.Cu") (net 3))
 (segment (start 99.4 59.8) (end 98.95 59.35) (width 0.25) (layer "B.Cu") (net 3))
 (segment (start 121.120974 51.836128) (end 118.963872 51.836128) (width 0.25) (layer "B.Cu") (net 3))
 (segment (start 90.15 47.8) (end 92.2 47.8) (width 0.25) (layer "B.Cu") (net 3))
 (segment (start 115.2835 49.2835) (end 116.82 49.2835) (width 0.25) (layer "F.Cu") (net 6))
 (segment (start 114.2 48.2) (end 115.2835 49.2835) (width 0.25) (layer "F.Cu") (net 6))
 (segment (start 111.95 39.35) (end 114.2 41.6) (width 0.25) (layer "F.Cu") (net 6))
 (segment (start 110.95 39.35) (end 111.95 39.35) (width 0.25) (layer "F.Cu") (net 6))
 (segment (start 110.95 39.35) (end 110.25 39.35) (width 0.25) (layer "F.Cu") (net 6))
 (segment (start 114.2 41.6) (end 114.2 48.2) (width 0.25) (layer "F.Cu") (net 6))
 (segment (start 106.17 52.55) (end 106.17 56.29) (width 0.25) (layer "F.Cu") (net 4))
 (segment (start 106.17 56.29) (end 111.15 61.27) (width 0.25) (layer "F.Cu") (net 4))
 (segment (start 96.2 75) (end 94.6 73.4) (width 1) (layer "B.Cu") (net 14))
 (segment (start 110.9 71.1) (end 110.3 70.5) (width 1) (layer "B.Cu") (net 14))
 (segment (start 116.78 71.1) (end 110.9 71.1) (width 1) (layer "B.Cu") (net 14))
 (segment (start 110.3 70.5) (end 105.8 75) (width 1) (layer "B.Cu") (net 14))
 (segment (start 105.8 75) (end 96.2 75) (width 1) (layer "B.Cu") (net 14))
 (segment (start 88.95 58.325) (end 88.95 54.22) (width 0.2) (layer "B.Cu") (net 17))
 (segment (start 95.7675 62.765) (end 95.835 62.765) (width 0.75) (layer "B.Cu") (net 17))
 (segment (start 96.73 60.13) (end 96.4 59.8) (width 0.2) (layer "B.Cu") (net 17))
 (segment (start 96.6 62) (end 96.5 62.1) (width 0.2) (layer "B.Cu") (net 17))
 (segment (start 96.4 59.8) (end 95 59.8) (width 0.2) (layer "B.Cu") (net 17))
 (segment (start 93.825 60.975) (end 91.6 60.975) (width 0.2) (layer "B.Cu") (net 17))
 (segment (start 95.835 62.765) (end 96.6 62) (width 0.75) (layer "B.Cu") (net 17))
 (segment (start 96.73 61.201396) (end 96.73 60.13) (width 0.2) (layer "B.Cu") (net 17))
 (segment (start 91.6 60.975) (end 88.95 58.325) (width 0.2) (layer "B.Cu") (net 17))
 (segment (start 95.831396 62.1) (end 96.73 61.201396) (width 0.2) (layer "B.Cu") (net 17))
 (segment (start 96.5 62.1) (end 95.831396 62.1) (width 0.2) (layer "B.Cu") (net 17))
 (segment (start 91.735 62.765) (end 90.6 63.9) (width 0.75) (layer "B.Cu") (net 17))
 (segment (start 95.7675 62.765) (end 91.735 62.765) (width 0.75) (layer "B.Cu") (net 17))
 (segment (start 95 59.8) (end 93.825 60.975) (width 0.2) (layer "B.Cu") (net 17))
 (segment (start 86.8 60.7) (end 85.45 59.35) (width 0.25) (layer "B.Cu") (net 16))
 (segment (start 95.2325 61.4) (end 86.8 61.4) (width 0.25) (layer "B.Cu") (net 16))
 (segment (start 95.7675 60.865) (end 95.2325 61.4) (width 0.25) (layer "B.Cu") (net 16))
 (segment (start 86.8 61.4) (end 86.8 60.7) (width 0.25) (layer "B.Cu") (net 16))
 (segment (start 117.023231 64.423231) (end 115 62.4) (width 0.2) (layer "B.Cu") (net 9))
 (segment (start 121.131352 64.423231) (end 117.023231 64.423231) (width 0.2) (layer "B.Cu") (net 9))
 (segment (start 115 62.4) (end 115 61.2635) (width 0.2) (layer "B.Cu") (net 9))
 (segment (start 115 61.2635) (end 116.82 59.4435) (width 0.2) (layer "B.Cu") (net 9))
 (segment (start 118.6 61.4) (end 118.2 61) (width 0.2) (layer "B.Cu") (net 10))
 (segment (start 121.015296 61.873231) (end 120.542065 61.4) (width 0.2) (layer "B.Cu") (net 10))
 (segment (start 118.2 58.2835) (end 116.82 56.9035) (width 0.2) (layer "B.Cu") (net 10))
 (segment (start 120.542065 61.4) (end 118.6 61.4) (width 0.2) (layer "B.Cu") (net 10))
 (segment (start 121.111352 61.873231) (end 121.015296 61.873231) (width 0.2) (layer "B.Cu") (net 10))
 (segment (start 118.2 61) (end 118.2 58.2835) (width 0.2) (layer "B.Cu") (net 10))
 (segment (start 118.2 57) (end 118.2 55.7435) (width 0.2) (layer "B.Cu") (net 11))
 (segment (start 120.549511 59.349511) (end 118.2 57) (width 0.2) (layer "B.Cu") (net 11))
 (segment (start 121.135519 59.349511) (end 120.549511 59.349511) (width 0.2) (layer "B.Cu") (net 11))
 (segment (start 118.2 55.7435) (end 116.82 54.3635) (width 0.2) (layer "B.Cu") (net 11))
 (segment (start 122.810441 54.310441) (end 125.7 57.2) (width 0.5) (layer "B.Cu") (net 13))
 (segment (start 121.135519 54.310441) (end 122.810441 54.310441) (width 0.5) (layer "B.Cu") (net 13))
 (segment (start 124.4 69.6) (end 124.4 71.1) (width 0.5) (layer "B.Cu") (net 18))
 (segment (start 121.8 67) (end 124.4 69.6) (width 0.5) (layer "B.Cu") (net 18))
 (segment (start 104.6 66) (end 105.6 67) (width 0.5) (layer "B.Cu") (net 18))
 (segment (start 111.85 37.8) (end 104.6 45.05) (width 0.5) (layer "B.Cu") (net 18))
 (segment (start 97.435 62.765) (end 95.2 65) (width 0.5) (layer "B.Cu") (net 18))
 (segment (start 104.6 45.05) (end 104.6 64.6) (width 0.5) (layer "B.Cu") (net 18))
 (segment (start 95.2 65) (end 94.61 65) (width 0.5) (layer "B.Cu") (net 18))
 (segment (start 104.6 64.6) (end 104.6 66) (width 0.5) (layer "B.Cu") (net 18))
 (segment (start 111.85 37.8) (end 111.85 40.25) (width 0.5) (layer "B.Cu") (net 18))
 (segment (start 105.6 67) (end 121.8 67) (width 0.5) (layer "B.Cu") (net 18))
 (segment (start 104.6 64.6) (end 99.8775 64.6) (width 0.5) (layer "B.Cu") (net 18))
 (segment (start 99.8775 64.6) (end 98.0425 62.765) (width 0.5) (layer "B.Cu") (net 18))
 (segment (start 111.85 40.25) (end 113.6 42) (width 0.5) (layer "B.Cu") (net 18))
 (segment (start 98.0425 62.765) (end 97.435 62.765) (width 0.5) (layer "B.Cu") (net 18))
 (segment (start 94.61 65) (end 93.31 66.3) (width 0.5) (layer "B.Cu") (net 18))
 (segment (start 100.4 55.7235) (end 101.58 56.9035) (width 0.25) (layer "B.Cu") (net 22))
 (segment (start 97.464481 51.200489) (end 98.416989 51.200489) (width 0.25) (layer "B.Cu") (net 22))
 (segment (start 100.4 53.935608) (end 100.4 55.7235) (width 0.25) (layer "B.Cu") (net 22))
 (segment (start 97.464481 51.200489) (end 97.664881 51.200489) (width 0.25) (layer "B.Cu") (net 22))
 (segment (start 97.664881 51.200489) (end 100.4 53.935608) (width 0.25) (layer "B.Cu") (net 22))
 (segment (start 99.8 54.4) (end 99.8 57.6635) (width 0.25) (layer "B.Cu") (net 21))
 (segment (start 99.079387 53.679387) (end 99.8 54.4) (width 0.25) (layer "B.Cu") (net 21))
 (segment (start 97.464481 53.679387) (end 99.079387 53.679387) (width 0.25) (layer "B.Cu") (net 21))
 (segment (start 99.8 57.6635) (end 101.58 59.4435) (width 0.25) (layer "B.Cu") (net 21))
 (segment (start 116.6715 51.675) (end 113.525 51.675) (width 0.25) (layer "F.Cu") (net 20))
 (segment (start 108.4 62.725) (end 104.8 62.725) (width 0.25) (layer "F.Cu") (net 20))
 (segment (start 102.65 58.275) (end 99.225 58.275) (width 0.25) (layer "F.Cu") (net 20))
 (segment (start 105.3 50.75) (end 104.85 51.2) (width 0.25) (layer "F.Cu") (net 20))
 (segment (start 116.82 51.8235) (end 116.6715 51.675) (width 0.25) (layer "F.Cu") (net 20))
 (segment (start 104.8 62.725) (end 103 60.925) (width 0.25) (layer "F.Cu") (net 20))
 (segment (start 103 60.925) (end 103 58.675) (width 0.25) (layer "F.Cu") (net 20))
 (segment (start 112.6 50.75) (end 105.3 50.75) (width 0.25) (layer "F.Cu") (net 20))
 (segment (start 104.85 56.55) (end 108.95 60.65) (width 0.25) (layer "F.Cu") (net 20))
 (segment (start 104.85 51.2) (end 104.85 56.55) (width 0.25) (layer "F.Cu") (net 20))
 (segment (start 108.95 60.65) (end 108.95 62.175) (width 0.25) (layer "F.Cu") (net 20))
 (segment (start 99.225 58.275) (end 97.575 56.625) (width 0.25) (layer "F.Cu") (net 20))
 (segment (start 103 58.675) (end 103.025 58.65) (width 0.25) (layer "F.Cu") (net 20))
 (segment (start 113.525 51.675) (end 112.6 50.75) (width 0.25) (layer "F.Cu") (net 20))
 (segment (start 103.025 58.65) (end 102.65 58.275) (width 0.25) (layer "F.Cu") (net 20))
 (segment (start 108.95 62.175) (end 108.4 62.725) (width 0.25) (layer "F.Cu") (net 20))
 (via (at 97.575 56.625) (size 0.8) (drill 0.4) (layers "F.Cu" "B.Cu") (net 20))
 (segment (start 97.464481 56.239559) (end 97.464481 57.064481) (width 0.25) (layer "B.Cu") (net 20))
 (segment (start 97.464481 56.239559) (end 98.376059 56.239559) (width 0.25) (layer "B.Cu") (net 20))
 (segment (start 103 52.9435) (end 101.58 54.3635) (width 0.2) (layer "B.Cu") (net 15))
 (segment (start 101.52 37.7) (end 103 39.18) (width 0.2) (layer "B.Cu") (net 15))
 (segment (start 103 39.18) (end 103 52.9435) (width 0.2) (layer "B.Cu") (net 15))
 (segment (start 125.863648 37.323231) (end 127.198231 37.323231) (width 0.25) (layer "F.Cu") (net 7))
 (segment (start 127.75 50.975) (end 127.025 51.7) (width 0.25) (layer "F.Cu") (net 7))
 (segment (start 128.3 41.9) (end 127.75 42.45) (width 0.25) (layer "F.Cu") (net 7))
 (segment (start 121.4 51.7) (end 120.925 52.175) (width 0.25) (layer "F.Cu") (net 7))
 (segment (start 127.198231 37.323231) (end 128.3 38.425) (width 0.25) (layer "F.Cu") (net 7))
 (segment (start 120.925 52.175) (end 120.925 59.025) (width 0.25) (layer "F.Cu") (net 7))
 (segment (start 120.925 59.025) (end 117.9665 61.9835) (width 0.25) (layer "F.Cu") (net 7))
 (segment (start 128.3 38.425) (end 128.3 41.9) (width 0.25) (layer "F.Cu") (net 7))
 (segment (start 117.9665 61.9835) (end 116.82 61.9835) (width 0.25) (layer "F.Cu") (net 7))
 (segment (start 127.025 51.7) (end 121.4 51.7) (width 0.25) (layer "F.Cu") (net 7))
 (segment (start 127.75 42.45) (end 127.75 50.975) (width 0.25) (layer "F.Cu") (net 7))
 (via (at 125.2 35) (size 0.8) (drill 0.4) (layers "F.Cu" "B.Cu") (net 8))
 (segment (start 103.75 60.425) (end 103.75 42.225) (width 0.25) (layer "B.Cu") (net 8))
 (segment (start 107.8 38.175) (end 107.8 33.7) (width 0.25) (layer "B.Cu") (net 8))
 (segment (start 103.75 42.225) (end 107.8 38.175) (width 0.25) (layer "B.Cu") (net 8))
 (segment (start 107.8 33.7) (end 108.575 32.925) (width 0.25) (layer "B.Cu") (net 8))
 (segment (start 123.125 32.925) (end 125.2 35) (width 0.25) (layer "B.Cu") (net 8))
 (segment (start 102.1915 61.9835) (end 103.75 60.425) (width 0.25) (layer "B.Cu") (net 8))
 (segment (start 101.58 61.9835) (end 102.1915 61.9835) (width 0.25) (layer "B.Cu") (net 8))
 (segment (start 108.575 32.925) (end 123.125 32.925) (width 0.25) (layer "B.Cu") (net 8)))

